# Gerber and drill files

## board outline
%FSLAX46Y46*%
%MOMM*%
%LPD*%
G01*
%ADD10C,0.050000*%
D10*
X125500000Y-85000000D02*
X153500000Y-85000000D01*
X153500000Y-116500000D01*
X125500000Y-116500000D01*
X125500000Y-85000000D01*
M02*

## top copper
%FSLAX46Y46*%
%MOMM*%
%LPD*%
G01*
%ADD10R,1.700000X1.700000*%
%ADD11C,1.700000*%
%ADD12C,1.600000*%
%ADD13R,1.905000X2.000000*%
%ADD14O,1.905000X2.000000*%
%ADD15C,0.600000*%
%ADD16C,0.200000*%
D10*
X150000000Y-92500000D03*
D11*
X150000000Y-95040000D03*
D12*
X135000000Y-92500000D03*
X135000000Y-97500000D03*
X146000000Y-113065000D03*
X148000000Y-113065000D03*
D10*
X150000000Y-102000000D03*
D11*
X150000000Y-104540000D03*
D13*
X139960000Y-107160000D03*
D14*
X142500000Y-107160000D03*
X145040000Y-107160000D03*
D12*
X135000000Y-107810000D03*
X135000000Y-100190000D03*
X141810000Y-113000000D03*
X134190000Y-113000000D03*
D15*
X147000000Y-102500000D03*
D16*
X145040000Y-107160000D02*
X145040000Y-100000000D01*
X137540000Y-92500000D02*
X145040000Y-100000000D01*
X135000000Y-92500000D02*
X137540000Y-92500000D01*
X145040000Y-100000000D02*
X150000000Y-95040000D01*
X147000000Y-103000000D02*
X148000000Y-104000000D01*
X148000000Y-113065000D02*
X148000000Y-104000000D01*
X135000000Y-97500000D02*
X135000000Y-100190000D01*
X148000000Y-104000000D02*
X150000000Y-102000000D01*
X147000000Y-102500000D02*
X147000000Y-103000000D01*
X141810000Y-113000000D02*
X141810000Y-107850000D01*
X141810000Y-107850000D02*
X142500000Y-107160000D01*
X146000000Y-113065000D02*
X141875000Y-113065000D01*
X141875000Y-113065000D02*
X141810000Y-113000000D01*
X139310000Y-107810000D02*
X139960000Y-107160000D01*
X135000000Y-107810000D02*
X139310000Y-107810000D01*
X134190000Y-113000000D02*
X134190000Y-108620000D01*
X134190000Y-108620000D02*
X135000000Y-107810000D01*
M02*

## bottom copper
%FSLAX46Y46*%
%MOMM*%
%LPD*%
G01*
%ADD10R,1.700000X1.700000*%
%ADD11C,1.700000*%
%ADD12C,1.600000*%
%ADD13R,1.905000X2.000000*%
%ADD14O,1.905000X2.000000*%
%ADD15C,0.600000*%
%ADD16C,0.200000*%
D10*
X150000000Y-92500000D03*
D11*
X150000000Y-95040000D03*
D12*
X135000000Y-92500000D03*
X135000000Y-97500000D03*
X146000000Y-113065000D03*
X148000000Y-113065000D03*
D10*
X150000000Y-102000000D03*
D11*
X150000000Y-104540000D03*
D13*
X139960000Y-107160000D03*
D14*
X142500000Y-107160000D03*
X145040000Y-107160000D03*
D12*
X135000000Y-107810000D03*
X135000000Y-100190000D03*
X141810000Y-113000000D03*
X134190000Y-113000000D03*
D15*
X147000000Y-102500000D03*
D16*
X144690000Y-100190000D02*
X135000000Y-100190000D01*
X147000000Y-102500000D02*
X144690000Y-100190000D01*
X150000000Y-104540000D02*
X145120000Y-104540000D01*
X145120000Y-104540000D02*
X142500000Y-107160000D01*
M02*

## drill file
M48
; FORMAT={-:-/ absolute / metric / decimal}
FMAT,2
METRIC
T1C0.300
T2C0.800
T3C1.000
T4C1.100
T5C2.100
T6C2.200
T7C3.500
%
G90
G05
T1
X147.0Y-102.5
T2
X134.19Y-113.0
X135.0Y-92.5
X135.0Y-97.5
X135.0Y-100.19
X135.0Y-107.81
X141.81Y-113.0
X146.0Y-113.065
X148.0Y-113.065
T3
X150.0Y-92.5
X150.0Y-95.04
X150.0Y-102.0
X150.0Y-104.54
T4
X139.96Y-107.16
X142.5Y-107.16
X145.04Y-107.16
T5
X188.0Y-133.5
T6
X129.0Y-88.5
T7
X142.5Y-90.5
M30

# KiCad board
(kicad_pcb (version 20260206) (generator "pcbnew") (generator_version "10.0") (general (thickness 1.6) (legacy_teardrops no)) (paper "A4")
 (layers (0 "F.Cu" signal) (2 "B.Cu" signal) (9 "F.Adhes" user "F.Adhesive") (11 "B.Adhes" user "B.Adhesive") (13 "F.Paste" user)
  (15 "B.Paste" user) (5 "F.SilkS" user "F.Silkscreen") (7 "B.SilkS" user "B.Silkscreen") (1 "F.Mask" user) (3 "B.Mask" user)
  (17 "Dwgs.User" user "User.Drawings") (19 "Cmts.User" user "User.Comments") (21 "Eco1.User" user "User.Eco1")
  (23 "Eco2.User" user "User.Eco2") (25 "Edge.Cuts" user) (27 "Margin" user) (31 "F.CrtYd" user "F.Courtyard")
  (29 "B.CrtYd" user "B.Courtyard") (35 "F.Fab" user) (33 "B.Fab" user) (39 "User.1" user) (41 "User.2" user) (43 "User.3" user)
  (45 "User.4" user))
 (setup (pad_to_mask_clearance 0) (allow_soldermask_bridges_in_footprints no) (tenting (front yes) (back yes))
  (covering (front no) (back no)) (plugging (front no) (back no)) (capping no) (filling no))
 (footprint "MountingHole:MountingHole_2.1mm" (layer "F.Cu") (at 188 133.5)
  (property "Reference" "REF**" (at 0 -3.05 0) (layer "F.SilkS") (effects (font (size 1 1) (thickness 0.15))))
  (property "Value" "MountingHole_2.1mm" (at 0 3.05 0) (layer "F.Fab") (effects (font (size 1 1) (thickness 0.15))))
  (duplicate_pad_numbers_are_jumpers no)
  (pad "" np_thru_hole circle (at 0 0) (size 2.1 2.1) (drill 2.1) (layers "*.Cu" "*.Mask")))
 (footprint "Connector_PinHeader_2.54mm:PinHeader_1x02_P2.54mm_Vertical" (layer "F.Cu") (at 150 92.5)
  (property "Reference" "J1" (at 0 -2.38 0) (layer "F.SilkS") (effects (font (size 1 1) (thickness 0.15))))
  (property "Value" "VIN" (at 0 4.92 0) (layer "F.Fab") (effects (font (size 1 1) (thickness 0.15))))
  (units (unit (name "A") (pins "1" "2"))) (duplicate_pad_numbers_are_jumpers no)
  (pad "1" thru_hole rect (at 0 0) (size 1.7 1.7) (drill 1) (layers "*.Cu" "*.Mask") (remove_unused_layers no) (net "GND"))
  (pad "2" thru_hole circle (at 0 2.54) (size 1.7 1.7) (drill 1) (layers "*.Cu" "*.Mask") (remove_unused_layers no) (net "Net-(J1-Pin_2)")))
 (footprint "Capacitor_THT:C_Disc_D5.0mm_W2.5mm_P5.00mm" (layer "F.Cu") (at 135 92.5 -90)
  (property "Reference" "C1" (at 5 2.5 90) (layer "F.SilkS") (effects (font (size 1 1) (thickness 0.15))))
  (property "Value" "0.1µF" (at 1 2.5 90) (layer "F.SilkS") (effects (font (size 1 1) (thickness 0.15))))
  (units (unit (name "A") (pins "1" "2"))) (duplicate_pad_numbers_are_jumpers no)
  (pad "1" thru_hole circle (at 0 0 270) (size 1.6 1.6) (drill 0.8) (layers "*.Cu" "*.Mask") (remove_unused_layers no)
   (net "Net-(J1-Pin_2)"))
  (pad "2" thru_hole circle (at 5 0 270) (size 1.6 1.6) (drill 0.8) (layers "*.Cu" "*.Mask") (remove_unused_layers no) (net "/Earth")))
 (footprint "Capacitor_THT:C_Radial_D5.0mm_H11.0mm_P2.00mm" (layer "F.Cu") (at 146 113.065)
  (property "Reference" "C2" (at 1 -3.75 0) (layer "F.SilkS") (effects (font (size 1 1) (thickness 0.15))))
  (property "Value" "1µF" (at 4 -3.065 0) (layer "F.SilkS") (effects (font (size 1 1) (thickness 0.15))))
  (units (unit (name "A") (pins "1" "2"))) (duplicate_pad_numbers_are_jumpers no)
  (pad "1" thru_hole circle (at 0 0) (size 1.6 1.6) (drill 0.8) (layers "*.Cu" "*.Mask") (remove_unused_layers no) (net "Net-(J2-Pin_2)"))
  (pad "2" thru_hole circle (at 2 0) (size 1.6 1.6) (drill 0.8) (layers "*.Cu" "*.Mask") (remove_unused_layers no) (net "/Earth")))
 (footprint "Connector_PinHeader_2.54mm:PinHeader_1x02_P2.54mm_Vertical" (layer "F.Cu") (at 150 102)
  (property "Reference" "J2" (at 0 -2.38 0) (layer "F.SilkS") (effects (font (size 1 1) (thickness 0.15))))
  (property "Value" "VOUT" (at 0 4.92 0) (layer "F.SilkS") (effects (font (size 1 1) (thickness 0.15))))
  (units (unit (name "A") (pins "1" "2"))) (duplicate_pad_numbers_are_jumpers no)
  (pad "1" thru_hole rect (at 0 0) (size 1.7 1.7) (drill 1) (layers "*.Cu" "*.Mask") (remove_unused_layers no) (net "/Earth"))
  (pad "2" thru_hole circle (at 0 2.54) (size 1.7 1.7) (drill 1) (layers "*.Cu" "*.Mask") (remove_unused_layers no) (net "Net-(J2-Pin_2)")))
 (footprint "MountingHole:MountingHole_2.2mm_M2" (layer "F.Cu") (at 129 88.5)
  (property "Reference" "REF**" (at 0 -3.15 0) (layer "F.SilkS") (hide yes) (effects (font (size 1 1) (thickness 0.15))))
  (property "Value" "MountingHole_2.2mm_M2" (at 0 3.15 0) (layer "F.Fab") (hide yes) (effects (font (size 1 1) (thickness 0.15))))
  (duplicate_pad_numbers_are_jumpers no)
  (pad "" np_thru_hole circle (at 0 0) (size 2.2 2.2) (drill 2.2) (layers "*.Cu" "*.Mask")))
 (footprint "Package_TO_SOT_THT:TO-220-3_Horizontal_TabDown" (layer "F.Cu") (at 139.96 107.16)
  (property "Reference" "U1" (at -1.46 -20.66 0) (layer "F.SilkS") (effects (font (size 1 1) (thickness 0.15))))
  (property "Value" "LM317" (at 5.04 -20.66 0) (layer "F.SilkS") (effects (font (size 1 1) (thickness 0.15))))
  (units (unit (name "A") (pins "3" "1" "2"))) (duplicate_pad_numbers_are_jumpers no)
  (pad "" np_thru_hole circle (at 2.54 -16.66) (size 3.5 3.5) (drill 3.5) (layers "*.Cu" "*.Mask"))
  (pad "1" thru_hole rect (at 0 0) (size 1.905 2) (drill 1.1) (layers "*.Cu" "*.Mask") (remove_unused_layers no) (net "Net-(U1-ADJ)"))
  (pad "2" thru_hole oval (at 2.54 0) (size 1.905 2) (drill 1.1) (layers "*.Cu" "*.Mask") (remove_unused_layers no) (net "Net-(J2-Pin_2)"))
  (pad "3" thru_hole oval (at 5.08 0) (size 1.905 2) (drill 1.1) (layers "*.Cu" "*.Mask") (remove_unused_layers no) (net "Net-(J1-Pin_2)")))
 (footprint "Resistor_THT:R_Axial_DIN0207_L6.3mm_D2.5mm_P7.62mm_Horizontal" (layer "F.Cu") (at 135 107.81 90)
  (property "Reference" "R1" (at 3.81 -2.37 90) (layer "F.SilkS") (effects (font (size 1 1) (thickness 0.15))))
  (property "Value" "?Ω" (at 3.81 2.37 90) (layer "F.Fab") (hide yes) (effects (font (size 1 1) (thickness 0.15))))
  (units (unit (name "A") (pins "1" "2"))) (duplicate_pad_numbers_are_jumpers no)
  (pad "1" thru_hole circle (at 0 0 90) (size 1.6 1.6) (drill 0.8) (layers "*.Cu" "*.Mask") (remove_unused_layers no) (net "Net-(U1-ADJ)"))
  (pad "2" thru_hole circle (at 7.62 0 90) (size 1.6 1.6) (drill 0.8) (layers "*.Cu" "*.Mask") (remove_unused_layers no) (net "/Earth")))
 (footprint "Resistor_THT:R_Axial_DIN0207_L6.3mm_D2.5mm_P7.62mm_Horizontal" (layer "F.Cu") (at 141.81 113 180)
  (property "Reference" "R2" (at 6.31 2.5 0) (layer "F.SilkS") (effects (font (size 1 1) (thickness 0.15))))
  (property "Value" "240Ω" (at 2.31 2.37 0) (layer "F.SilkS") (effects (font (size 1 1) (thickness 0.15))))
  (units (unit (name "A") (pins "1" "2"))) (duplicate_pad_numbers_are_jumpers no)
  (pad "1" thru_hole circle (at 0 0 180) (size 1.6 1.6) (drill 0.8) (layers "*.Cu" "*.Mask") (remove_unused_layers no)
   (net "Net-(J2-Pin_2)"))
  (pad "2" thru_hole circle (at 7.62 0 180) (size 1.6 1.6) (drill 0.8) (layers "*.Cu" "*.Mask") (remove_unused_layers no)
   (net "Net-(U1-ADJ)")))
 (gr_rect (start 125.5 85) (end 153.5 116.5) (stroke (width 0.05) (type default)) (fill no) (layer "Edge.Cuts"))
 (segment (start 145.04 107.16) (end 145.04 100) (width 0.2) (layer "F.Cu") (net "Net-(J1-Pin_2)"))
 (segment (start 137.54 92.5) (end 145.04 100) (width 0.2) (layer "F.Cu") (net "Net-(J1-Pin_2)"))
 (segment (start 135 92.5) (end 137.54 92.5) (width 0.2) (layer "F.Cu") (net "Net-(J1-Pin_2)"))
 (segment (start 145.04 100) (end 150 95.04) (width 0.2) (layer "F.Cu") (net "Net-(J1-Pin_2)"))
 (segment (start 147 103) (end 148 104) (width 0.2) (layer "F.Cu") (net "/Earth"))
 (segment (start 148 113.065) (end 148 104) (width 0.2) (layer "F.Cu") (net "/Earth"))
 (segment (start 135 97.5) (end 135 100.19) (width 0.2) (layer "F.Cu") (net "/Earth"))
 (segment (start 148 104) (end 150 102) (width 0.2) (layer "F.Cu") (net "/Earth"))
 (segment (start 147 102.5) (end 147 103) (width 0.2) (layer "F.Cu") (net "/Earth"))
 (via (at 147 102.5) (size 0.6) (drill 0.3) (layers "F.Cu" "B.Cu") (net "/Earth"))
 (segment (start 144.69 100.19) (end 135 100.19) (width 0.2) (layer "B.Cu") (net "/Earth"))
 (segment (start 147 102.5) (end 144.69 100.19) (width 0.2) (layer "B.Cu") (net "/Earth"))
 (segment (start 141.81 113) (end 141.81 107.85) (width 0.2) (layer "F.Cu") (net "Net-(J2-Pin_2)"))
 (segment (start 141.81 107.85) (end 142.5 107.16) (width 0.2) (layer "F.Cu") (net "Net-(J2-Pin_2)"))
 (segment (start 146 113.065) (end 141.875 113.065) (width 0.2) (layer "F.Cu") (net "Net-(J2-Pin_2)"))
 (segment (start 141.875 113.065) (end 141.81 113) (width 0.2) (layer "F.Cu") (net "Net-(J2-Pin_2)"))
 (segment (start 150 104.54) (end 145.12 104.54) (width 0.2) (layer "B.Cu") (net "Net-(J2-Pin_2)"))
 (segment (start 145.12 104.54) (end 142.5 107.16) (width 0.2) (layer "B.Cu") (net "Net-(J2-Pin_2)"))
 (segment (start 139.31 107.81) (end 139.96 107.16) (width 0.2) (layer "F.Cu") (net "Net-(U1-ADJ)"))
 (segment (start 135 107.81) (end 139.31 107.81) (width 0.2) (layer "F.Cu") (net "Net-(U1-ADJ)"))
 (segment (start 134.19 113) (end 134.19 108.62) (width 0.2) (layer "F.Cu") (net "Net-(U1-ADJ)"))
 (segment (start 134.19 108.62) (end 135 107.81) (width 0.2) (layer "F.Cu") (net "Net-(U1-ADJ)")))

